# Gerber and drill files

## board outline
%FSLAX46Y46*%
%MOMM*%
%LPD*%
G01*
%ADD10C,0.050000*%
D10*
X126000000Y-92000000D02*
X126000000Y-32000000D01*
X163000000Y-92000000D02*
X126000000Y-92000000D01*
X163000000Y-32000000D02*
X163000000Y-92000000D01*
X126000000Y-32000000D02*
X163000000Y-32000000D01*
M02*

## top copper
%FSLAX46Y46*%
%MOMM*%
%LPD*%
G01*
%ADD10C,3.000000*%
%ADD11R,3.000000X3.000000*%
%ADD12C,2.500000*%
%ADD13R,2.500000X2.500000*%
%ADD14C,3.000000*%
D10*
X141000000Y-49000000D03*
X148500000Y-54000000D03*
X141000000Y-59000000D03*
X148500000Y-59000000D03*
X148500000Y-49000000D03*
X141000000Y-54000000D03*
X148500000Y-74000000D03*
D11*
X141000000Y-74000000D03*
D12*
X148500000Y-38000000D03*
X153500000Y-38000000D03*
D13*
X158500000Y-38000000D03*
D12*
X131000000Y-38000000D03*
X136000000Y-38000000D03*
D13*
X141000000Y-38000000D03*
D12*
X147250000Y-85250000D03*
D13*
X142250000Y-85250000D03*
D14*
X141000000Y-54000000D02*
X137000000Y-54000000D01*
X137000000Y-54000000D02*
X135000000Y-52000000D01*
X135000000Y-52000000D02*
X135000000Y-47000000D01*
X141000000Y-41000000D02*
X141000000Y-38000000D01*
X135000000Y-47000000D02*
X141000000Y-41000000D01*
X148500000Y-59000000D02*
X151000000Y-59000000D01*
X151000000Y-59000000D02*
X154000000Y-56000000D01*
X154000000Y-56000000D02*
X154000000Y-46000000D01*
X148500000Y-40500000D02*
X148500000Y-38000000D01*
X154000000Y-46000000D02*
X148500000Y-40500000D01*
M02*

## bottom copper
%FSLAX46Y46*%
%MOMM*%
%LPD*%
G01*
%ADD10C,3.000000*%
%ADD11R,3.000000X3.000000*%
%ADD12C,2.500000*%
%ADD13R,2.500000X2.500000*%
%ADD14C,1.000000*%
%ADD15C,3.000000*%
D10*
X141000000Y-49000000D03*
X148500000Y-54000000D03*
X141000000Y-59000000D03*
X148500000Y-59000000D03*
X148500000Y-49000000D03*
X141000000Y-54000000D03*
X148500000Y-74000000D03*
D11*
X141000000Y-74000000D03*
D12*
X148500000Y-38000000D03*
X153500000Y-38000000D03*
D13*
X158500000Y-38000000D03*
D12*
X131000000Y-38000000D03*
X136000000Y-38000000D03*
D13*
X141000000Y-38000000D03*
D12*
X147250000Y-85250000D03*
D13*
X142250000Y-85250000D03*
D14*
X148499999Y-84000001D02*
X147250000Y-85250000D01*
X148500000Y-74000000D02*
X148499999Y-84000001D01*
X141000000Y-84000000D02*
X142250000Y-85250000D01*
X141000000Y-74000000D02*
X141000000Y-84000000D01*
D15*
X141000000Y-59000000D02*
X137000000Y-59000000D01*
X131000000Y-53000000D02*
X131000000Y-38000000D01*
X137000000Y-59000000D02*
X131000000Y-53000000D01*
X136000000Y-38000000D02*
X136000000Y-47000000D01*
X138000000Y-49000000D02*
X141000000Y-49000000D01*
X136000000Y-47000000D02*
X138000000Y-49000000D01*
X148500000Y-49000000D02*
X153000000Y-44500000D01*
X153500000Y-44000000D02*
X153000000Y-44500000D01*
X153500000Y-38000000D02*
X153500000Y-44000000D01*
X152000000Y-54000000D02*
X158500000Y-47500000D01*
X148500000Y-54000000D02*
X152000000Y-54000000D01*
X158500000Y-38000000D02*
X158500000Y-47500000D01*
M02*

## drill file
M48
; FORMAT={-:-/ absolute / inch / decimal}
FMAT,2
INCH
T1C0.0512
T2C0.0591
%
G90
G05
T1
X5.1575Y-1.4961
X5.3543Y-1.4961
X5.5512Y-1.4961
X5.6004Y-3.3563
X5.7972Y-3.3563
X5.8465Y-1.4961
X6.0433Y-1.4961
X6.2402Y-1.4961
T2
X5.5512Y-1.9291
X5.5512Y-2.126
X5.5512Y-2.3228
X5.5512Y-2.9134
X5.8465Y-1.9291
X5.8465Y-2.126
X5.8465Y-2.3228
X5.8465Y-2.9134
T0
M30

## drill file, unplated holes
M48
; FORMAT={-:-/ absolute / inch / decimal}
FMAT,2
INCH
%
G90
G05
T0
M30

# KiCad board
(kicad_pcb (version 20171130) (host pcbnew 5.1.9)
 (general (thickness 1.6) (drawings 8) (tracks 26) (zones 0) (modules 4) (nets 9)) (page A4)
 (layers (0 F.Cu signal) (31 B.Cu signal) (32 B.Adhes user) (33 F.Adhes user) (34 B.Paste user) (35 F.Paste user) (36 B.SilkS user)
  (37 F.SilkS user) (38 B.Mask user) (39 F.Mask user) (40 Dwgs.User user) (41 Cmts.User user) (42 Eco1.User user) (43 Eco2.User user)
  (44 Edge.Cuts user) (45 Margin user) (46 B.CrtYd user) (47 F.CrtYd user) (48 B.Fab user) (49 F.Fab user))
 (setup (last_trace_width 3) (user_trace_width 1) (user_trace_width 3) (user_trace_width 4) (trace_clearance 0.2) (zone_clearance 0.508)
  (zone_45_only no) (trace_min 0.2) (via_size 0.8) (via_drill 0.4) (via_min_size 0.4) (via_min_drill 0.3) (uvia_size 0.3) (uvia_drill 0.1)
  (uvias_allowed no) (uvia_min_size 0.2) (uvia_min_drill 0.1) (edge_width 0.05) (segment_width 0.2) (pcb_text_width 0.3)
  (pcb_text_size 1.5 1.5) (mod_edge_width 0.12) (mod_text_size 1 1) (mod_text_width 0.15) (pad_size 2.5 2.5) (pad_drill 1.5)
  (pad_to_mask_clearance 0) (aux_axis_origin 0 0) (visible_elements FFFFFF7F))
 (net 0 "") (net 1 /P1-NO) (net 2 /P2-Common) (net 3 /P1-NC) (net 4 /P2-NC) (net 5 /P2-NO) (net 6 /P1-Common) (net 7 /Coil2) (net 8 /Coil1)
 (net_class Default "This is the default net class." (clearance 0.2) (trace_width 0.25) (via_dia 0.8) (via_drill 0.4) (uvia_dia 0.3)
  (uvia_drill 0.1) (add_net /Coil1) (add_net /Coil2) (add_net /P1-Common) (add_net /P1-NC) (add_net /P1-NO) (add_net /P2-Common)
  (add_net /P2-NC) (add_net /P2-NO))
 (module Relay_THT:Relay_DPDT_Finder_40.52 (layer F.Cu) (at 141 74 90)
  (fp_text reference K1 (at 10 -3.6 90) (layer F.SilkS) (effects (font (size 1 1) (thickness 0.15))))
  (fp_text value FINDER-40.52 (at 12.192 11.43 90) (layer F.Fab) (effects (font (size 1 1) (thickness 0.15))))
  (pad 14 thru_hole circle (at 25 0 90) (size 3 3) (drill 1.5) (layers *.Cu *.Mask) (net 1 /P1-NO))
  (pad 21 thru_hole circle (at 20 7.5 90) (size 3 3) (drill 1.5) (layers *.Cu *.Mask) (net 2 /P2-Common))
  (pad 12 thru_hole circle (at 15 0 90) (size 3 3) (drill 1.5) (layers *.Cu *.Mask) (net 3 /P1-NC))
  (pad 22 thru_hole circle (at 15 7.5 90) (size 3 3) (drill 1.5) (layers *.Cu *.Mask) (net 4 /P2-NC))
  (pad 24 thru_hole circle (at 25 7.5 90) (size 3 3) (drill 1.5) (layers *.Cu *.Mask) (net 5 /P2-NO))
  (pad 11 thru_hole circle (at 20 0 90) (size 3 3) (drill 1.5) (layers *.Cu *.Mask) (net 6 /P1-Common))
  (pad A2 thru_hole circle (at 0 7.5 90) (size 3 3) (drill 1.5) (layers *.Cu *.Mask) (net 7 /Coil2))
  (pad A1 thru_hole rect (at 0 0 90) (size 3 3) (drill 1.5) (layers *.Cu *.Mask) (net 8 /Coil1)))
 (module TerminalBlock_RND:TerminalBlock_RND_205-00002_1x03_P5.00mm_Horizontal (layer F.Cu) (at 158.5 38 180)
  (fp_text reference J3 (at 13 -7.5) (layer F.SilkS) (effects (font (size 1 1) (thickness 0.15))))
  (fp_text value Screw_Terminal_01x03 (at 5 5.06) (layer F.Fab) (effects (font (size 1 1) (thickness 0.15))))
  (pad 3 thru_hole circle (at 10 0 180) (size 2.5 2.5) (drill 1.3) (layers *.Cu *.Mask) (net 4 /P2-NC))
  (pad 2 thru_hole circle (at 5 0 180) (size 2.5 2.5) (drill 1.3) (layers *.Cu *.Mask) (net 5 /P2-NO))
  (pad 1 thru_hole rect (at 0 0 180) (size 2.5 2.5) (drill 1.3) (layers *.Cu *.Mask) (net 2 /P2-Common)))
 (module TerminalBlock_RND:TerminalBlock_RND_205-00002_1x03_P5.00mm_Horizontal (layer F.Cu) (at 141 38 180)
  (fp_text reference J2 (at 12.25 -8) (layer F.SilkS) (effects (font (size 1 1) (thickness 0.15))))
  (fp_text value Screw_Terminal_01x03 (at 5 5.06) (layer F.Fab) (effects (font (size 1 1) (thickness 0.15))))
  (pad 3 thru_hole circle (at 10 0 180) (size 2.5 2.5) (drill 1.3) (layers *.Cu *.Mask) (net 3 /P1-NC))
  (pad 2 thru_hole circle (at 5 0 180) (size 2.5 2.5) (drill 1.3) (layers *.Cu *.Mask) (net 1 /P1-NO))
  (pad 1 thru_hole rect (at 0 0 180) (size 2.5 2.5) (drill 1.3) (layers *.Cu *.Mask) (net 6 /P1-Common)))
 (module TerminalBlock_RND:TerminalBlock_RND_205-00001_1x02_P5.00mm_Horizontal (layer F.Cu) (at 142.25 85.25)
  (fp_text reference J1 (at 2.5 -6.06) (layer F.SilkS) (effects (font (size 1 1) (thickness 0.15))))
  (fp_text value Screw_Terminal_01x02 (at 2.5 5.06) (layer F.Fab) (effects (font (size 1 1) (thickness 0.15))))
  (pad 2 thru_hole circle (at 5 0) (size 2.5 2.5) (drill 1.3) (layers *.Cu *.Mask) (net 7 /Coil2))
  (pad 1 thru_hole rect (at 0 0) (size 2.5 2.5) (drill 1.3) (layers *.Cu *.Mask) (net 8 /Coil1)))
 (gr_line (start 126 92) (end 126 32) (layer Edge.Cuts) (width 0.05))
 (gr_line (start 163 92) (end 126 92) (layer Edge.Cuts) (width 0.05))
 (gr_line (start 163 32) (end 163 92) (layer Edge.Cuts) (width 0.05))
 (gr_line (start 126 32) (end 163 32) (layer Edge.Cuts) (width 0.05))
 (segment (start 148.499999 84.000001) (end 147.25 85.25) (width 1) (layer B.Cu) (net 7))
 (segment (start 148.5 74) (end 148.499999 84.000001) (width 1) (layer B.Cu) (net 7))
 (segment (start 141 84) (end 142.25 85.25) (width 1) (layer B.Cu) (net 8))
 (segment (start 141 74) (end 141 84) (width 1) (layer B.Cu) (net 8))
 (segment (start 141 59) (end 137 59) (width 3) (layer B.Cu) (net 3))
 (segment (start 131 53) (end 131 38) (width 3) (layer B.Cu) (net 3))
 (segment (start 137 59) (end 131 53) (width 3) (layer B.Cu) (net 3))
 (segment (start 136 38) (end 136 47) (width 3) (layer B.Cu) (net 1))
 (segment (start 138 49) (end 141 49) (width 3) (layer B.Cu) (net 1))
 (segment (start 136 47) (end 138 49) (width 3) (layer B.Cu) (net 1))
 (segment (start 141 54) (end 137 54) (width 3) (layer F.Cu) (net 6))
 (segment (start 137 54) (end 135 52) (width 3) (layer F.Cu) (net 6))
 (segment (start 135 52) (end 135 47) (width 3) (layer F.Cu) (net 6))
 (segment (start 141 41) (end 141 38) (width 3) (layer F.Cu) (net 6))
 (segment (start 135 47) (end 141 41) (width 3) (layer F.Cu) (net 6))
 (segment (start 148.5 59) (end 151 59) (width 3) (layer F.Cu) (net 4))
 (segment (start 151 59) (end 154 56) (width 3) (layer F.Cu) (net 4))
 (segment (start 154 56) (end 154 46) (width 3) (layer F.Cu) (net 4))
 (segment (start 148.5 40.5) (end 148.5 38) (width 3) (layer F.Cu) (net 4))
 (segment (start 154 46) (end 148.5 40.5) (width 3) (layer F.Cu) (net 4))
 (segment (start 148.5 49) (end 153 44.5) (width 3) (layer B.Cu) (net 5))
 (segment (start 153.5 44) (end 153 44.5) (width 3) (layer B.Cu) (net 5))
 (segment (start 153.5 38) (end 153.5 44) (width 3) (layer B.Cu) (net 5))
 (segment (start 152 54) (end 158.5 47.5) (width 3) (layer B.Cu) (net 2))
 (segment (start 148.5 54) (end 152 54) (width 3) (layer B.Cu) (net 2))
 (segment (start 158.5 38) (end 158.5 47.5) (width 3) (layer B.Cu) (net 2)))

